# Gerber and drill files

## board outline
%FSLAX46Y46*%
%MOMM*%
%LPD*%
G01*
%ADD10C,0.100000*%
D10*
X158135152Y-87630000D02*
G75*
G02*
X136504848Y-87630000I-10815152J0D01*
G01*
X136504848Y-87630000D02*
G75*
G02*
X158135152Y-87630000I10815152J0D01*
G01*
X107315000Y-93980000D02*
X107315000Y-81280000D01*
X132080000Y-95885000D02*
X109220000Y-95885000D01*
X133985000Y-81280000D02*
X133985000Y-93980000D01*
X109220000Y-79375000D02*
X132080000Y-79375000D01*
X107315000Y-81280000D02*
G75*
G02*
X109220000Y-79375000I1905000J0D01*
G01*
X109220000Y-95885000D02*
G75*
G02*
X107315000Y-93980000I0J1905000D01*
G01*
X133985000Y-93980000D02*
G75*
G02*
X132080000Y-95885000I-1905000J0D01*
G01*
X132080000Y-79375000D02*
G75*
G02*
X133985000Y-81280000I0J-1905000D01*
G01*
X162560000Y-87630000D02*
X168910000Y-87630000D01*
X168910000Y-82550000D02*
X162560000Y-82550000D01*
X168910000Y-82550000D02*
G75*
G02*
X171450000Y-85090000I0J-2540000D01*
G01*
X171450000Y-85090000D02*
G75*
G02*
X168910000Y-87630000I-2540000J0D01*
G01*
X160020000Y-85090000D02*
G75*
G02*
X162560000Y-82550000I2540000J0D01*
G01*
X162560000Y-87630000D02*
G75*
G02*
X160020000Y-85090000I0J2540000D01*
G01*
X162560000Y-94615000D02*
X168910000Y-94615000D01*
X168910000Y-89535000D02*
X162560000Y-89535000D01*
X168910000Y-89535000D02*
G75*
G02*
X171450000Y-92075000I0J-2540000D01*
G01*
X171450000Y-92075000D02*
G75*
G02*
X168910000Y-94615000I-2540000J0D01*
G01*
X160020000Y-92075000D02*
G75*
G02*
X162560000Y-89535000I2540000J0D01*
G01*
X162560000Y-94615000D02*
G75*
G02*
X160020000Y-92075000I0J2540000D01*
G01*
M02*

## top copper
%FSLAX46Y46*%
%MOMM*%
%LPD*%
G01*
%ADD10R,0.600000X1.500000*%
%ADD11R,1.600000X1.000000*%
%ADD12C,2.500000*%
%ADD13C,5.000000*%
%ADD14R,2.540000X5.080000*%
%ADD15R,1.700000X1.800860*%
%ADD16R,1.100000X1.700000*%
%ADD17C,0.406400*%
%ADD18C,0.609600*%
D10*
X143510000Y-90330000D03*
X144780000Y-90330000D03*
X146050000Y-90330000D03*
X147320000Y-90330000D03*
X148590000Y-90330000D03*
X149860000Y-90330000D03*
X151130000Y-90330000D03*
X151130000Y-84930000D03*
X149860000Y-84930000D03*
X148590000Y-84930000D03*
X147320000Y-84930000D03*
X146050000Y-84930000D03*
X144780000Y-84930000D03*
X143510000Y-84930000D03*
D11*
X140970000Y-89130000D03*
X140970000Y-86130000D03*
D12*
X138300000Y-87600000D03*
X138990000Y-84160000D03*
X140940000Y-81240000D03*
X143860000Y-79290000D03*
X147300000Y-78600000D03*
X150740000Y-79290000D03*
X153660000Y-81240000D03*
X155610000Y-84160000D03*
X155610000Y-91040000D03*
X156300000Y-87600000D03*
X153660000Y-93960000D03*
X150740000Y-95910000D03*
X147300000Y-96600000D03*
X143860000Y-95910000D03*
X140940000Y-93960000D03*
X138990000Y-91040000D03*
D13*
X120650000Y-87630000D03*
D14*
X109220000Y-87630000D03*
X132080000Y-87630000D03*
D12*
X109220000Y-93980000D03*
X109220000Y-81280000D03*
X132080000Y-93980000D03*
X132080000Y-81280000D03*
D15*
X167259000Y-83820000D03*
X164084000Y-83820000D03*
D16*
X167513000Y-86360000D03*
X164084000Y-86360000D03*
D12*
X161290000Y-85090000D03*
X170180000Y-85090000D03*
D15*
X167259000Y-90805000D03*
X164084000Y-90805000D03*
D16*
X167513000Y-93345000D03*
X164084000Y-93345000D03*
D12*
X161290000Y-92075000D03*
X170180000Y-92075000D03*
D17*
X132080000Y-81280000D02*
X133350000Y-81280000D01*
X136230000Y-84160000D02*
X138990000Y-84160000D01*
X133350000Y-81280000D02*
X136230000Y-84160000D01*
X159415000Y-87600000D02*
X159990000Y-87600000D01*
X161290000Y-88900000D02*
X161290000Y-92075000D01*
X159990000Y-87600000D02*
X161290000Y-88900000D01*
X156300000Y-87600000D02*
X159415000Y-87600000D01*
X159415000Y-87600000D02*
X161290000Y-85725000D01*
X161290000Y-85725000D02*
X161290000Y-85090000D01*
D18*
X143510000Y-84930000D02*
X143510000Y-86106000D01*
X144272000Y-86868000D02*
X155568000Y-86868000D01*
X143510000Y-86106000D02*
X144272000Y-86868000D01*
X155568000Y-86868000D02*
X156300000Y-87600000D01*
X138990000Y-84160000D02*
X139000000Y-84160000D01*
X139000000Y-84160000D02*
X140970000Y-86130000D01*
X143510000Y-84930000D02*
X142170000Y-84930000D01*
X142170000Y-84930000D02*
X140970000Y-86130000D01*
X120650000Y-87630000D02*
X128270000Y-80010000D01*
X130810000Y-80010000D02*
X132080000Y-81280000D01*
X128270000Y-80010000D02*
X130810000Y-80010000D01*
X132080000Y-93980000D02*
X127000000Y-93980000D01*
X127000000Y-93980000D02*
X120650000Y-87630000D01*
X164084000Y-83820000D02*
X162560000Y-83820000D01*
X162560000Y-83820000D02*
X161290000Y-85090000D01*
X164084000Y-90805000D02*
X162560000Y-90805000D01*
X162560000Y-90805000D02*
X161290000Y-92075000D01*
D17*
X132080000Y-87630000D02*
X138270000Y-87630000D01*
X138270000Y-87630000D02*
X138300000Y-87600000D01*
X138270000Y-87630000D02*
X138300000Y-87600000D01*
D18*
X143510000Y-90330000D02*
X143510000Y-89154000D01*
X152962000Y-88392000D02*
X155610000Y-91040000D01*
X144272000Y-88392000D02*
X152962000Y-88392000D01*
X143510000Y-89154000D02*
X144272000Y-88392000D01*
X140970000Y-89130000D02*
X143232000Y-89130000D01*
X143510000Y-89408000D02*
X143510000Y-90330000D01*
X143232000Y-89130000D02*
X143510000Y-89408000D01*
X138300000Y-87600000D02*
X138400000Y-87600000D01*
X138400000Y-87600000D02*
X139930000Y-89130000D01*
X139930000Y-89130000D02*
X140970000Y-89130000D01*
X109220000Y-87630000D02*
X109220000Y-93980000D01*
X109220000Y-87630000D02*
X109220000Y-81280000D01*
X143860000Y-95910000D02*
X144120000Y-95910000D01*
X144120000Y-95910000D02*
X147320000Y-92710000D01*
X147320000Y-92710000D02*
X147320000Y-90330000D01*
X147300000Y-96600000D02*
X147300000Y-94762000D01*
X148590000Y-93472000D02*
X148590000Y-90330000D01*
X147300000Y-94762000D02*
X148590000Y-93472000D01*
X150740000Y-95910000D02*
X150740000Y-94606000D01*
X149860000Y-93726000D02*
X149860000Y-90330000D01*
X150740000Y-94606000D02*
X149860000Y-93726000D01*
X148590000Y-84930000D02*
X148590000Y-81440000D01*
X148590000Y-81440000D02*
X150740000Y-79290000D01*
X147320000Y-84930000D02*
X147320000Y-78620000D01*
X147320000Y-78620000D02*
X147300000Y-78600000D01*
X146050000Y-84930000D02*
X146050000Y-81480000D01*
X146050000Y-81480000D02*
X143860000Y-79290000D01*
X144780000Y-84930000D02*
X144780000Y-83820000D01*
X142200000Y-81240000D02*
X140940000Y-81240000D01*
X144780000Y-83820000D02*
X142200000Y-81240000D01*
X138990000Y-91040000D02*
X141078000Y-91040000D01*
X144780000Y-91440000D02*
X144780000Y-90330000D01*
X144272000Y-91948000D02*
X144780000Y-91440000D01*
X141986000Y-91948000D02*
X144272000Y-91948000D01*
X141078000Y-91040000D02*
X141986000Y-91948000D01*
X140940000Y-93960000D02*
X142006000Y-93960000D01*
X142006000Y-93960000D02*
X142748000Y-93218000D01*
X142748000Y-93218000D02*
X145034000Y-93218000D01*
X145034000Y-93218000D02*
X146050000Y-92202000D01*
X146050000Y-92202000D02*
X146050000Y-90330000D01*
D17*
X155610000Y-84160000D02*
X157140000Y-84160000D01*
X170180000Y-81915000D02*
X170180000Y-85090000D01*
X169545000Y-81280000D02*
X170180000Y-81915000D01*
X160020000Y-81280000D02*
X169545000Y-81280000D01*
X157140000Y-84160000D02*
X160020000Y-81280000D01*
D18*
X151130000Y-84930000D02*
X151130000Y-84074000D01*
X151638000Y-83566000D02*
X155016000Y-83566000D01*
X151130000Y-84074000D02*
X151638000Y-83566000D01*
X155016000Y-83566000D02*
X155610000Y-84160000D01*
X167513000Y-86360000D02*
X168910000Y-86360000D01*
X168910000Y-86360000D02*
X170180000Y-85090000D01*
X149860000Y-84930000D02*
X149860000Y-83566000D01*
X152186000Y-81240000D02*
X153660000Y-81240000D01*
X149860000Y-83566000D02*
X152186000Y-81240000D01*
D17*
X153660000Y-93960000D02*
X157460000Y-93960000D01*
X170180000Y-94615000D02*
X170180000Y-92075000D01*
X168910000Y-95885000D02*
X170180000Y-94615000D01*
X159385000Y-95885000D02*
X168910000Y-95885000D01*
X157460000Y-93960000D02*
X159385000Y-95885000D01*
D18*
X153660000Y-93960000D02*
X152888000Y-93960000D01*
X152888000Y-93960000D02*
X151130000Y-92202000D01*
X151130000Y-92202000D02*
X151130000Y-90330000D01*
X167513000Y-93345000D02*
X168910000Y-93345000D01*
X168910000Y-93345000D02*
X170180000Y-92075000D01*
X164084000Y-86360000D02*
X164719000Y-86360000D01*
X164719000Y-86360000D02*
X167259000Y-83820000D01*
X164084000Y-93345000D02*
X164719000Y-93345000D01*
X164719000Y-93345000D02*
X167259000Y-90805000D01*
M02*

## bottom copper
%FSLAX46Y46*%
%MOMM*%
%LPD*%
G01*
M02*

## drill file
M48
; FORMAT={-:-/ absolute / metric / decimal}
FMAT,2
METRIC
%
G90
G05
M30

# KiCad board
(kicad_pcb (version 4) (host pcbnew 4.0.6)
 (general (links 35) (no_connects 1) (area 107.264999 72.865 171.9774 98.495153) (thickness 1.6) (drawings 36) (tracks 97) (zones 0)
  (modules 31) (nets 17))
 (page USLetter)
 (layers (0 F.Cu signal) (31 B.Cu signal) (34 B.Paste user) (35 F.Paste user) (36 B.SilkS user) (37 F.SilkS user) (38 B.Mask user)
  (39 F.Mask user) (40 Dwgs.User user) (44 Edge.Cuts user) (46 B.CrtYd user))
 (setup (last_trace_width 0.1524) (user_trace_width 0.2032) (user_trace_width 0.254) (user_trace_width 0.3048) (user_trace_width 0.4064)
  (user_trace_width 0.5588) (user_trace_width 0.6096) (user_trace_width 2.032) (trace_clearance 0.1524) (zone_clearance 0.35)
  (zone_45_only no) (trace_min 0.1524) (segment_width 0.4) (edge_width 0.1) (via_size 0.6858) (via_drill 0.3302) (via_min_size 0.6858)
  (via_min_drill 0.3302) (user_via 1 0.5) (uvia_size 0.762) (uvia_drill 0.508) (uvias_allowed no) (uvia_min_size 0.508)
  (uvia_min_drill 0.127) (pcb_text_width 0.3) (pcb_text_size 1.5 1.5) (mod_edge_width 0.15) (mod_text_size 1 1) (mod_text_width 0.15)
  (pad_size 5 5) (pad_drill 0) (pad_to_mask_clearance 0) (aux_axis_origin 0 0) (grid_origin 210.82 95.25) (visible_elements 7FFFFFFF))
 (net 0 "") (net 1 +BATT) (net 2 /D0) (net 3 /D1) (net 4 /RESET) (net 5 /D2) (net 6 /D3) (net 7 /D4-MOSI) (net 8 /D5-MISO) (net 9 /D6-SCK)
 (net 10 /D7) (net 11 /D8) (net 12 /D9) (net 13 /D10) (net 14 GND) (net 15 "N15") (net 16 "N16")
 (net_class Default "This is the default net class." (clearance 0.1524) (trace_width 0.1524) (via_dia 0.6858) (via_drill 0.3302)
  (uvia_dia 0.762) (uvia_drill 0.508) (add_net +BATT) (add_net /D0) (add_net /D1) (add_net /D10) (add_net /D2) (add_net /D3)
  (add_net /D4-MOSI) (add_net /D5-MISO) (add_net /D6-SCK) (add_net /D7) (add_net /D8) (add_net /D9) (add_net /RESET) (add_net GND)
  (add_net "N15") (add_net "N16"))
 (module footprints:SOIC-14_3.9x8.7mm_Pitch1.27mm (layer F.Cu) (at 147.32 87.63 90)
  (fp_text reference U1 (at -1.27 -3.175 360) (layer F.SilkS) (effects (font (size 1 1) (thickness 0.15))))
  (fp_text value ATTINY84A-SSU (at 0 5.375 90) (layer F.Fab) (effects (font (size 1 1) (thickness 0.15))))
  (pad 1 smd rect (at -2.7 -3.81 90) (size 1.5 0.6) (layers F.Cu F.Paste F.Mask) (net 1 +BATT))
  (pad 2 smd rect (at -2.7 -2.54 90) (size 1.5 0.6) (layers F.Cu F.Paste F.Mask) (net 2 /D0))
  (pad 3 smd rect (at -2.7 -1.27 90) (size 1.5 0.6) (layers F.Cu F.Paste F.Mask) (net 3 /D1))
  (pad 4 smd rect (at -2.7 0 90) (size 1.5 0.6) (layers F.Cu F.Paste F.Mask) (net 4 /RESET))
  (pad 5 smd rect (at -2.7 1.27 90) (size 1.5 0.6) (layers F.Cu F.Paste F.Mask) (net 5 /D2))
  (pad 6 smd rect (at -2.7 2.54 90) (size 1.5 0.6) (layers F.Cu F.Paste F.Mask) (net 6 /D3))
  (pad 7 smd rect (at -2.7 3.81 90) (size 1.5 0.6) (layers F.Cu F.Paste F.Mask) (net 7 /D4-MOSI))
  (pad 8 smd rect (at 2.7 3.81 90) (size 1.5 0.6) (layers F.Cu F.Paste F.Mask) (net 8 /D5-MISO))
  (pad 9 smd rect (at 2.7 2.54 90) (size 1.5 0.6) (layers F.Cu F.Paste F.Mask) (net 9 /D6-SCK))
  (pad 10 smd rect (at 2.7 1.27 90) (size 1.5 0.6) (layers F.Cu F.Paste F.Mask) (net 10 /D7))
  (pad 11 smd rect (at 2.7 0 90) (size 1.5 0.6) (layers F.Cu F.Paste F.Mask) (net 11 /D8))
  (pad 12 smd rect (at 2.7 -1.27 90) (size 1.5 0.6) (layers F.Cu F.Paste F.Mask) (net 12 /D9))
  (pad 13 smd rect (at 2.7 -2.54 90) (size 1.5 0.6) (layers F.Cu F.Paste F.Mask) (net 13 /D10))
  (pad 14 smd rect (at 2.7 -3.81 90) (size 1.5 0.6) (layers F.Cu F.Paste F.Mask) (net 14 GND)))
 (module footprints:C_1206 (layer F.Cu) (at 140.97 87.63 90)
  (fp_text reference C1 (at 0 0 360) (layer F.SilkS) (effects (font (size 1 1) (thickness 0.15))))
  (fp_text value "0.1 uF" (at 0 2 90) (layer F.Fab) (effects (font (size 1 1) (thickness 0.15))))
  (pad 1 smd rect (at -1.5 0 90) (size 1 1.6) (layers F.Cu F.Paste F.Mask) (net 1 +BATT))
  (pad 2 smd rect (at 1.5 0 90) (size 1 1.6) (layers F.Cu F.Paste F.Mask) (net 14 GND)))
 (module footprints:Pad (layer F.Cu) (at 138.3 87.6)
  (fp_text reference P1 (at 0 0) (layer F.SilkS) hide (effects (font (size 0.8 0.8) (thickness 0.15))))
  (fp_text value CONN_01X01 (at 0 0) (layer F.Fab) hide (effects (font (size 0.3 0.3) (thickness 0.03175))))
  (pad 1 smd circle (at 0 0) (size 2.5 2.5) (layers F.Cu F.Paste F.Mask) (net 1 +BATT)))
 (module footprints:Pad (layer F.Cu) (at 138.99 84.16)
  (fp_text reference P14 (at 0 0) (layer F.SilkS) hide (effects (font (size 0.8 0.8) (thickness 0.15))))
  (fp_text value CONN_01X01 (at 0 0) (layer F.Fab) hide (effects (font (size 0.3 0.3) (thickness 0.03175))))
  (pad 1 smd circle (at 0 0) (size 2.5 2.5) (layers F.Cu F.Paste F.Mask) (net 14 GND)))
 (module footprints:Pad (layer F.Cu) (at 140.94 81.24)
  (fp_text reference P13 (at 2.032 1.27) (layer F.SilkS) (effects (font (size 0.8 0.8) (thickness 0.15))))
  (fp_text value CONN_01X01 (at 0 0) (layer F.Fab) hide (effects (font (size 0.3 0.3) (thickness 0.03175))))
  (pad 1 smd circle (at 0 0) (size 2.5 2.5) (layers F.Cu F.Paste F.Mask) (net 13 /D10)))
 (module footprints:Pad (layer F.Cu) (at 143.86 79.29)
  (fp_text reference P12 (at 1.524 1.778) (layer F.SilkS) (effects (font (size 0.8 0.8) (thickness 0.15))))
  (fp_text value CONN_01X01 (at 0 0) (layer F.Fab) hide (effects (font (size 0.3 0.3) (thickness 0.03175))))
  (pad 1 smd circle (at 0 0) (size 2.5 2.5) (layers F.Cu F.Paste F.Mask) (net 12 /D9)))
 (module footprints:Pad (layer F.Cu) (at 147.3 78.6)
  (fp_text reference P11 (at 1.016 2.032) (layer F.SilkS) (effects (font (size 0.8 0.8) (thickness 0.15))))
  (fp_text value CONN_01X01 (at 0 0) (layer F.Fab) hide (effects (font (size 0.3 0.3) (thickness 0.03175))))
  (pad 1 smd circle (at 0 0) (size 2.5 2.5) (layers F.Cu F.Paste F.Mask) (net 11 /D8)))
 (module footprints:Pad (layer F.Cu) (at 150.74 79.29)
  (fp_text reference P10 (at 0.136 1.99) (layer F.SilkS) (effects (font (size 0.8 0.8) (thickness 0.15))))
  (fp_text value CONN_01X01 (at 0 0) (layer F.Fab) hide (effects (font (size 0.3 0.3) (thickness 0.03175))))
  (pad 1 smd circle (at 0 0) (size 2.5 2.5) (layers F.Cu F.Paste F.Mask) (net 10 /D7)))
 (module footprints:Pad (layer F.Cu) (at 153.66 81.24)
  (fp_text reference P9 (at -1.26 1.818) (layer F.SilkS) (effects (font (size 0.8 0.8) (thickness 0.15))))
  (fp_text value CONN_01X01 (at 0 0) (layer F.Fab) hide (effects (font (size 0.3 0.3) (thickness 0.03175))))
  (pad 1 smd circle (at 0 0) (size 2.5 2.5) (layers F.Cu F.Paste F.Mask) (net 9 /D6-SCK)))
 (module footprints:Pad (layer F.Cu) (at 155.61 84.16)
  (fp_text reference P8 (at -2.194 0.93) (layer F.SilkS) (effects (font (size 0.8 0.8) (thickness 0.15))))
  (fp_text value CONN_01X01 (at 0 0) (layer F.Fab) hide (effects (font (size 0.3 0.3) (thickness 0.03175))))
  (pad 1 smd circle (at 0 0) (size 2.5 2.5) (layers F.Cu F.Paste F.Mask) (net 8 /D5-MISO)))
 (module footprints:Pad (layer F.Cu) (at 155.61 91.04)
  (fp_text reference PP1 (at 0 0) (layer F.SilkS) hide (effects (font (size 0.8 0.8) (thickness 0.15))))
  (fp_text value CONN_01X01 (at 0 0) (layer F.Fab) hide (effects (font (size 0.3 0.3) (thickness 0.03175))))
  (pad 1 smd circle (at 0 0) (size 2.5 2.5) (layers F.Cu F.Paste F.Mask) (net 1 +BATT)))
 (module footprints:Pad (layer F.Cu) (at 156.3 87.6)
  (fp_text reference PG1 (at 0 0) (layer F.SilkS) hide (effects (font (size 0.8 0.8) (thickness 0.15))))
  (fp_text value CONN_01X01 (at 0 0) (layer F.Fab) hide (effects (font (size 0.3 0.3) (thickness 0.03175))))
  (pad 1 smd circle (at 0 0) (size 2.5 2.5) (layers F.Cu F.Paste F.Mask) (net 14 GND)))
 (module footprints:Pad (layer F.Cu) (at 153.66 93.96)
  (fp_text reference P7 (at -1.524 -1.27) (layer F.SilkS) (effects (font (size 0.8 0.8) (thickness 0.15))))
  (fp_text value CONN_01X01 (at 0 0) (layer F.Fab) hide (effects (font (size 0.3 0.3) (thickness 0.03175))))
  (pad 1 smd circle (at 0 0) (size 2.5 2.5) (layers F.Cu F.Paste F.Mask) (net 7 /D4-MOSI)))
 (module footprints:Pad (layer F.Cu) (at 150.74 95.91)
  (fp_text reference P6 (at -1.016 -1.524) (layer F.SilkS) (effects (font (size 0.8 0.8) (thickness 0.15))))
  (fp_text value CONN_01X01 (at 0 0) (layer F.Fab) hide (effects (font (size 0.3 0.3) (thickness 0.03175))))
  (pad 1 smd circle (at 0 0) (size 2.5 2.5) (layers F.Cu F.Paste F.Mask) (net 6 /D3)))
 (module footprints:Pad (layer F.Cu) (at 147.3 96.6)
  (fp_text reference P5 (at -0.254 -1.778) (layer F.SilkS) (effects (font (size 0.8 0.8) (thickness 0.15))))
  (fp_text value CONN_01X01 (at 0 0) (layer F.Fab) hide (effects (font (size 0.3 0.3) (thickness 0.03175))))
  (pad 1 smd circle (at 0 0) (size 2.5 2.5) (layers F.Cu F.Paste F.Mask) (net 5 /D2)))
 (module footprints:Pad (layer F.Cu) (at 143.86 95.91)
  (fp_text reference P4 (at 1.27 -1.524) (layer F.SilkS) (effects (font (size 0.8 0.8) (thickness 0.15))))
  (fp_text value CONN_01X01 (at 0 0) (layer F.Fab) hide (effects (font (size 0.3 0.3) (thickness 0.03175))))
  (pad 1 smd circle (at 0 0) (size 2.5 2.5) (layers F.Cu F.Paste F.Mask) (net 4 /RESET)))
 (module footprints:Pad (layer F.Cu) (at 140.94 93.96)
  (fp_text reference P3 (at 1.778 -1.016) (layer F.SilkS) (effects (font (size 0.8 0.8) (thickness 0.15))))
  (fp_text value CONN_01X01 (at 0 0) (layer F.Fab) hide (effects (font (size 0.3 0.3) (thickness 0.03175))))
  (pad 1 smd circle (at 0 0) (size 2.5 2.5) (layers F.Cu F.Paste F.Mask) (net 3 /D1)))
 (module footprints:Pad (layer F.Cu) (at 138.99 91.04)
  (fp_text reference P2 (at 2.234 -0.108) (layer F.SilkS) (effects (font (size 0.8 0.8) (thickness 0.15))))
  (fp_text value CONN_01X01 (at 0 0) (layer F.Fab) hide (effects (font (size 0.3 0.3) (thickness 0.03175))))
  (pad 1 smd circle (at 0 0) (size 2.5 2.5) (layers F.Cu F.Paste F.Mask) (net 2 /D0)))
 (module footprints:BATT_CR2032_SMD (layer F.Cu) (at 120.65 87.63)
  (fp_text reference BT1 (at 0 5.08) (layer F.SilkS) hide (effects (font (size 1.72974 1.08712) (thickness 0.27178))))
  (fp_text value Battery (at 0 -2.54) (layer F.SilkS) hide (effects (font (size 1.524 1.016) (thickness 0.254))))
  (pad 2 smd circle (at 0 0) (size 5 5) (layers F.Cu F.Paste F.Mask) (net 14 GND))
  (pad 1 smd rect (at -11.43 0) (size 2.54 5.08) (layers F.Cu F.Paste F.Mask) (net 1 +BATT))
  (pad 1 smd rect (at 11.43 0) (size 2.54 5.08) (layers F.Cu F.Paste F.Mask) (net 1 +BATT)))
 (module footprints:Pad (layer F.Cu) (at 109.22 93.98)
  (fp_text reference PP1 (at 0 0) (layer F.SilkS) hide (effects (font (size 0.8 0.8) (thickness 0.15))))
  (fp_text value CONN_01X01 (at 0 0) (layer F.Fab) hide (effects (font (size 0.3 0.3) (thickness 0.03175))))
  (pad 1 smd circle (at 0 0) (size 2.5 2.5) (layers F.Cu F.Paste F.Mask) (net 1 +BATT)))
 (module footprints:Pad (layer F.Cu) (at 109.22 81.28)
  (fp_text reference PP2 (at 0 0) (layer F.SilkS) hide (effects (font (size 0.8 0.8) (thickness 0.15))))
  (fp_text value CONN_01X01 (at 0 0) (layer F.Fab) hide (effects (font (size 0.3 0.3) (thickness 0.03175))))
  (pad 1 smd circle (at 0 0) (size 2.5 2.5) (layers F.Cu F.Paste F.Mask) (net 1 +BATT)))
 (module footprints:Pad (layer F.Cu) (at 132.08 93.98)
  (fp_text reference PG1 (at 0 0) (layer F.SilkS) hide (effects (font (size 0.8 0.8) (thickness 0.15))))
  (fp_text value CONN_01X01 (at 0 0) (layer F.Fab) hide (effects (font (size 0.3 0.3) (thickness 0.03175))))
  (pad 1 smd circle (at 0 0) (size 2.5 2.5) (layers F.Cu F.Paste F.Mask) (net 14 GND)))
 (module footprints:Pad (layer F.Cu) (at 132.08 81.28)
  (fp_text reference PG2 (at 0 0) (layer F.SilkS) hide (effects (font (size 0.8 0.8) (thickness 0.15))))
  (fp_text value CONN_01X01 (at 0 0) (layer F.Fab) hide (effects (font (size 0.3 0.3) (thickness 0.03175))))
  (pad 1 smd circle (at 0 0) (size 2.5 2.5) (layers F.Cu F.Paste F.Mask) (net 14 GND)))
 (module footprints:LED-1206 (layer F.Cu) (at 165.735 83.82)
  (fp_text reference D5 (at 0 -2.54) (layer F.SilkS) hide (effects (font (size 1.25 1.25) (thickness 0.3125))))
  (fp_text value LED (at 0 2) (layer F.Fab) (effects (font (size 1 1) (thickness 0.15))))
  (pad 2 smd rect (at 1.524 0 180) (size 1.7 1.80086) (layers F.Cu F.Paste F.Mask) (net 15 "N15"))
  (pad 1 smd rect (at -1.651 0 180) (size 1.7 1.80086) (layers F.Cu F.Paste F.Mask) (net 14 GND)))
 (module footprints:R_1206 (layer F.Cu) (at 165.735 86.36 180)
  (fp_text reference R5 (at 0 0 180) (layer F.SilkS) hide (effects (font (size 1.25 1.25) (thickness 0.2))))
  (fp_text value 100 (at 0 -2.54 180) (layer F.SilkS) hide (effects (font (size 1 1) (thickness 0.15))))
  (pad 1 smd rect (at -1.778 0 180) (size 1.1 1.7) (layers F.Cu F.Paste F.Mask) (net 8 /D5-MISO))
  (pad 2 smd rect (at 1.651 0 180) (size 1.1 1.7) (layers F.Cu F.Paste F.Mask) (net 15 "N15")))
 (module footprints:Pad (layer F.Cu) (at 161.29 85.09 90)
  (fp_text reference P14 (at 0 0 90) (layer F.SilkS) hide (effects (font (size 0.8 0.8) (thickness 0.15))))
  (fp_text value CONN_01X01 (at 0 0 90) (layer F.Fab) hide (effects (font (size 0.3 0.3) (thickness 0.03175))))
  (pad 1 smd circle (at 0 0 90) (size 2.5 2.5) (layers F.Cu F.Paste F.Mask) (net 14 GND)))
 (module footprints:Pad (layer F.Cu) (at 170.18 85.09 90)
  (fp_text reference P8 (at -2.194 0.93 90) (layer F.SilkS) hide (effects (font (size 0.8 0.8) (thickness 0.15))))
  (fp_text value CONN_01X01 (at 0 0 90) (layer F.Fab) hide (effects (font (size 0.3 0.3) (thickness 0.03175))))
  (pad 1 smd circle (at 0 0 90) (size 2.5 2.5) (layers F.Cu F.Paste F.Mask) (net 8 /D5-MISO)))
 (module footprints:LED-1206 (layer F.Cu) (at 165.735 90.805)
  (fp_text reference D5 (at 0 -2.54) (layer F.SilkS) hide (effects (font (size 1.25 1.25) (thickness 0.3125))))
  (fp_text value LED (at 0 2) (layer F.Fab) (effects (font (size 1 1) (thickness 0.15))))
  (pad 2 smd rect (at 1.524 0 180) (size 1.7 1.80086) (layers F.Cu F.Paste F.Mask) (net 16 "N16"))
  (pad 1 smd rect (at -1.651 0 180) (size 1.7 1.80086) (layers F.Cu F.Paste F.Mask) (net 14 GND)))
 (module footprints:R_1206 (layer F.Cu) (at 165.735 93.345 180)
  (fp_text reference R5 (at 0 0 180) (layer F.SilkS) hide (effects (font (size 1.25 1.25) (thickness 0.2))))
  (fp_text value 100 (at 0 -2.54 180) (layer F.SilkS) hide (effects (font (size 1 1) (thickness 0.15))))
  (pad 1 smd rect (at -1.778 0 180) (size 1.1 1.7) (layers F.Cu F.Paste F.Mask) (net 7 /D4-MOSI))
  (pad 2 smd rect (at 1.651 0 180) (size 1.1 1.7) (layers F.Cu F.Paste F.Mask) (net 16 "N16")))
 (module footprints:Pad (layer F.Cu) (at 161.29 92.075 90)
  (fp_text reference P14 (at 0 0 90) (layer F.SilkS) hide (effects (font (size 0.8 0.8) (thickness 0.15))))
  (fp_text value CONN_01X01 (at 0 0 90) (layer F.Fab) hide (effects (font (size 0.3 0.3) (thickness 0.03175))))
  (pad 1 smd circle (at 0 0 90) (size 2.5 2.5) (layers F.Cu F.Paste F.Mask) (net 14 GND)))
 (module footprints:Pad (layer F.Cu) (at 170.18 92.075 90)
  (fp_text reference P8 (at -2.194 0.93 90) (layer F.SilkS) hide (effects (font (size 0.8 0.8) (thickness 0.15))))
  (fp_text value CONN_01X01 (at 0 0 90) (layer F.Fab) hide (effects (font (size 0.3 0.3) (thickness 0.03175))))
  (pad 1 smd circle (at 0 0 90) (size 2.5 2.5) (layers F.Cu F.Paste F.Mask) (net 7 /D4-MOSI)))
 (gr_circle (center 147.32 87.63) (end 149.098 98.298) (layer Edge.Cuts) (width 0.1))
 (gr_line (start 107.315 93.98) (end 107.315 81.28) (angle 90) (layer Edge.Cuts) (width 0.1))
 (gr_line (start 132.08 95.885) (end 109.22 95.885) (angle 90) (layer Edge.Cuts) (width 0.1))
 (gr_line (start 133.985 81.28) (end 133.985 93.98) (angle 90) (layer Edge.Cuts) (width 0.1))
 (gr_line (start 109.22 79.375) (end 132.08 79.375) (angle 90) (layer Edge.Cuts) (width 0.1))
 (gr_arc (start 109.22 81.28) (end 107.315 81.28) (angle 90) (layer Edge.Cuts) (width 0.1))
 (gr_arc (start 109.22 93.98) (end 109.22 95.885) (angle 90) (layer Edge.Cuts) (width 0.1))
 (gr_arc (start 132.08 93.98) (end 133.985 93.98) (angle 90) (layer Edge.Cuts) (width 0.1))
 (gr_arc (start 132.08 81.28) (end 132.08 79.375) (angle 90) (layer Edge.Cuts) (width 0.1))
 (gr_line (start 162.56 87.63) (end 168.91 87.63) (angle 90) (layer Edge.Cuts) (width 0.1))
 (gr_line (start 168.91 82.55) (end 162.56 82.55) (angle 90) (layer Edge.Cuts) (width 0.1))
 (gr_arc (start 168.91 85.09) (end 168.91 82.55) (angle 90) (layer Edge.Cuts) (width 0.1))
 (gr_arc (start 168.91 85.09) (end 171.45 85.09) (angle 90) (layer Edge.Cuts) (width 0.1))
 (gr_arc (start 162.56 85.09) (end 160.02 85.09) (angle 90) (layer Edge.Cuts) (width 0.1))
 (gr_arc (start 162.56 85.09) (end 162.56 87.63) (angle 90) (layer Edge.Cuts) (width 0.1))
 (gr_line (start 162.56 94.615) (end 168.91 94.615) (angle 90) (layer Edge.Cuts) (width 0.1))
 (gr_line (start 168.91 89.535) (end 162.56 89.535) (angle 90) (layer Edge.Cuts) (width 0.1))
 (gr_arc (start 168.91 92.075) (end 168.91 89.535) (angle 90) (layer Edge.Cuts) (width 0.1))
 (gr_arc (start 168.91 92.075) (end 171.45 92.075) (angle 90) (layer Edge.Cuts) (width 0.1))
 (gr_arc (start 162.56 92.075) (end 160.02 92.075) (angle 90) (layer Edge.Cuts) (width 0.1))
 (gr_arc (start 162.56 92.075) (end 162.56 94.615) (angle 90) (layer Edge.Cuts) (width 0.1))
 (segment (start 132.08 81.28) (end 133.35 81.28) (width 0.4064) (layer F.Cu) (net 14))
 (segment (start 136.23 84.16) (end 138.99 84.16) (width 0.4064) (layer F.Cu) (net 14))
 (segment (start 133.35 81.28) (end 136.23 84.16) (width 0.4064) (layer F.Cu) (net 14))
 (segment (start 159.415 87.6) (end 159.99 87.6) (width 0.4064) (layer F.Cu) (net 14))
 (segment (start 161.29 88.9) (end 161.29 92.075) (width 0.4064) (layer F.Cu) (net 14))
 (segment (start 159.99 87.6) (end 161.29 88.9) (width 0.4064) (layer F.Cu) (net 14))
 (segment (start 156.3 87.6) (end 159.415 87.6) (width 0.4064) (layer F.Cu) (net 14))
 (segment (start 159.415 87.6) (end 161.29 85.725) (width 0.4064) (layer F.Cu) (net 14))
 (segment (start 161.29 85.725) (end 161.29 85.09) (width 0.4064) (layer F.Cu) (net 14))
 (segment (start 143.51 84.93) (end 143.51 86.106) (width 0.6096) (layer F.Cu) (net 14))
 (segment (start 144.272 86.868) (end 155.568 86.868) (width 0.6096) (layer F.Cu) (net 14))
 (segment (start 143.51 86.106) (end 144.272 86.868) (width 0.6096) (layer F.Cu) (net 14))
 (segment (start 155.568 86.868) (end 156.3 87.6) (width 0.6096) (layer F.Cu) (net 14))
 (segment (start 138.99 84.16) (end 139 84.16) (width 0.6096) (layer F.Cu) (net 14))
 (segment (start 139 84.16) (end 140.97 86.13) (width 0.6096) (layer F.Cu) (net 14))
 (segment (start 143.51 84.93) (end 142.17 84.93) (width 0.6096) (layer F.Cu) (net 14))
 (segment (start 142.17 84.93) (end 140.97 86.13) (width 0.6096) (layer F.Cu) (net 14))
 (segment (start 120.65 87.63) (end 128.27 80.01) (width 0.6096) (layer F.Cu) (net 14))
 (segment (start 130.81 80.01) (end 132.08 81.28) (width 0.6096) (layer F.Cu) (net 14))
 (segment (start 128.27 80.01) (end 130.81 80.01) (width 0.6096) (layer F.Cu) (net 14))
 (segment (start 132.08 93.98) (end 127 93.98) (width 0.6096) (layer F.Cu) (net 14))
 (segment (start 127 93.98) (end 120.65 87.63) (width 0.6096) (layer F.Cu) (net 14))
 (segment (start 164.084 83.82) (end 162.56 83.82) (width 0.6096) (layer F.Cu) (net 14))
 (segment (start 162.56 83.82) (end 161.29 85.09) (width 0.6096) (layer F.Cu) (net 14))
 (segment (start 164.084 90.805) (end 162.56 90.805) (width 0.6096) (layer F.Cu) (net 14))
 (segment (start 162.56 90.805) (end 161.29 92.075) (width 0.6096) (layer F.Cu) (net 14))
 (segment (start 132.08 87.63) (end 138.27 87.63) (width 0.4064) (layer F.Cu) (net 1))
 (segment (start 138.27 87.63) (end 138.3 87.6) (width 0.4064) (layer F.Cu) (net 1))
 (segment (start 138.27 87.63) (end 138.3 87.6) (width 0.4064) (layer F.Cu) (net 1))
 (segment (start 143.51 90.33) (end 143.51 89.154) (width 0.6096) (layer F.Cu) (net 1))
 (segment (start 152.962 88.392) (end 155.61 91.04) (width 0.6096) (layer F.Cu) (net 1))
 (segment (start 144.272 88.392) (end 152.962 88.392) (width 0.6096) (layer F.Cu) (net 1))
 (segment (start 143.51 89.154) (end 144.272 88.392) (width 0.6096) (layer F.Cu) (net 1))
 (segment (start 140.97 89.13) (end 143.232 89.13) (width 0.6096) (layer F.Cu) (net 1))
 (segment (start 143.51 89.408) (end 143.51 90.33) (width 0.6096) (layer F.Cu) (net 1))
 (segment (start 143.232 89.13) (end 143.51 89.408) (width 0.6096) (layer F.Cu) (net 1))
 (segment (start 138.3 87.6) (end 138.4 87.6) (width 0.6096) (layer F.Cu) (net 1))
 (segment (start 138.4 87.6) (end 139.93 89.13) (width 0.6096) (layer F.Cu) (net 1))
 (segment (start 139.93 89.13) (end 140.97 89.13) (width 0.6096) (layer F.Cu) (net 1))
 (segment (start 109.22 87.63) (end 109.22 93.98) (width 0.6096) (layer F.Cu) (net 1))
 (segment (start 109.22 87.63) (end 109.22 81.28) (width 0.6096) (layer F.Cu) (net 1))
 (segment (start 143.86 95.91) (end 144.12 95.91) (width 0.6096) (layer F.Cu) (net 4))
 (segment (start 144.12 95.91) (end 147.32 92.71) (width 0.6096) (layer F.Cu) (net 4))
 (segment (start 147.32 92.71) (end 147.32 90.33) (width 0.6096) (layer F.Cu) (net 4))
 (segment (start 147.3 96.6) (end 147.3 94.762) (width 0.6096) (layer F.Cu) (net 5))
 (segment (start 148.59 93.472) (end 148.59 90.33) (width 0.6096) (layer F.Cu) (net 5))
 (segment (start 147.3 94.762) (end 148.59 93.472) (width 0.6096) (layer F.Cu) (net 5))
 (segment (start 150.74 95.91) (end 150.74 94.606) (width 0.6096) (layer F.Cu) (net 6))
 (segment (start 149.86 93.726) (end 149.86 90.33) (width 0.6096) (layer F.Cu) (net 6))
 (segment (start 150.74 94.606) (end 149.86 93.726) (width 0.6096) (layer F.Cu) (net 6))
 (segment (start 148.59 84.93) (end 148.59 81.44) (width 0.6096) (layer F.Cu) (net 10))
 (segment (start 148.59 81.44) (end 150.74 79.29) (width 0.6096) (layer F.Cu) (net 10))
 (segment (start 147.32 84.93) (end 147.32 78.62) (width 0.6096) (layer F.Cu) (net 11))
 (segment (start 147.32 78.62) (end 147.3 78.6) (width 0.6096) (layer F.Cu) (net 11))
 (segment (start 146.05 84.93) (end 146.05 81.48) (width 0.6096) (layer F.Cu) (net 12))
 (segment (start 146.05 81.48) (end 143.86 79.29) (width 0.6096) (layer F.Cu) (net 12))
 (segment (start 144.78 84.93) (end 144.78 83.82) (width 0.6096) (layer F.Cu) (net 13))
 (segment (start 142.2 81.24) (end 140.94 81.24) (width 0.6096) (layer F.Cu) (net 13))
 (segment (start 144.78 83.82) (end 142.2 81.24) (width 0.6096) (layer F.Cu) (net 13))
 (segment (start 138.99 91.04) (end 141.078 91.04) (width 0.6096) (layer F.Cu) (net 2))
 (segment (start 144.78 91.44) (end 144.78 90.33) (width 0.6096) (layer F.Cu) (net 2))
 (segment (start 144.272 91.948) (end 144.78 91.44) (width 0.6096) (layer F.Cu) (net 2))
 (segment (start 141.986 91.948) (end 144.272 91.948) (width 0.6096) (layer F.Cu) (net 2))
 (segment (start 141.078 91.04) (end 141.986 91.948) (width 0.6096) (layer F.Cu) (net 2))
 (segment (start 140.94 93.96) (end 142.006 93.96) (width 0.6096) (layer F.Cu) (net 3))
 (segment (start 142.006 93.96) (end 142.748 93.218) (width 0.6096) (layer F.Cu) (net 3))
 (segment (start 142.748 93.218) (end 145.034 93.218) (width 0.6096) (layer F.Cu) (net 3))
 (segment (start 145.034 93.218) (end 146.05 92.202) (width 0.6096) (layer F.Cu) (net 3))
 (segment (start 146.05 92.202) (end 146.05 90.33) (width 0.6096) (layer F.Cu) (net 3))
 (segment (start 155.61 84.16) (end 157.14 84.16) (width 0.4064) (layer F.Cu) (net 8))
 (segment (start 170.18 81.915) (end 170.18 85.09) (width 0.4064) (layer F.Cu) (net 8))
 (segment (start 169.545 81.28) (end 170.18 81.915) (width 0.4064) (layer F.Cu) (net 8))
 (segment (start 160.02 81.28) (end 169.545 81.28) (width 0.4064) (layer F.Cu) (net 8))
 (segment (start 157.14 84.16) (end 160.02 81.28) (width 0.4064) (layer F.Cu) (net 8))
 (segment (start 151.13 84.93) (end 151.13 84.074) (width 0.6096) (layer F.Cu) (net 8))
 (segment (start 151.638 83.566) (end 155.016 83.566) (width 0.6096) (layer F.Cu) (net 8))
 (segment (start 151.13 84.074) (end 151.638 83.566) (width 0.6096) (layer F.Cu) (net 8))
 (segment (start 155.016 83.566) (end 155.61 84.16) (width 0.6096) (layer F.Cu) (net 8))
 (segment (start 167.513 86.36) (end 168.91 86.36) (width 0.6096) (layer F.Cu) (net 8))
 (segment (start 168.91 86.36) (end 170.18 85.09) (width 0.6096) (layer F.Cu) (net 8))
 (segment (start 149.86 84.93) (end 149.86 83.566) (width 0.6096) (layer F.Cu) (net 9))
 (segment (start 152.186 81.24) (end 153.66 81.24) (width 0.6096) (layer F.Cu) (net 9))
 (segment (start 149.86 83.566) (end 152.186 81.24) (width 0.6096) (layer F.Cu) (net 9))
 (segment (start 153.66 93.96) (end 157.46 93.96) (width 0.4064) (layer F.Cu) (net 7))
 (segment (start 170.18 94.615) (end 170.18 92.075) (width 0.4064) (layer F.Cu) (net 7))
 (segment (start 168.91 95.885) (end 170.18 94.615) (width 0.4064) (layer F.Cu) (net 7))
 (segment (start 159.385 95.885) (end 168.91 95.885) (width 0.4064) (layer F.Cu) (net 7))
 (segment (start 157.46 93.96) (end 159.385 95.885) (width 0.4064) (layer F.Cu) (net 7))
 (segment (start 153.66 93.96) (end 152.888 93.96) (width 0.6096) (layer F.Cu) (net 7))
 (segment (start 152.888 93.96) (end 151.13 92.202) (width 0.6096) (layer F.Cu) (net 7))
 (segment (start 151.13 92.202) (end 151.13 90.33) (width 0.6096) (layer F.Cu) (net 7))
 (segment (start 167.513 93.345) (end 168.91 93.345) (width 0.6096) (layer F.Cu) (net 7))
 (segment (start 168.91 93.345) (end 170.18 92.075) (width 0.6096) (layer F.Cu) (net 7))
 (segment (start 164.084 86.36) (end 164.719 86.36) (width 0.6096) (layer F.Cu) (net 15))
 (segment (start 164.719 86.36) (end 167.259 83.82) (width 0.6096) (layer F.Cu) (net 15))
 (segment (start 164.084 93.345) (end 164.719 93.345) (width 0.6096) (layer F.Cu) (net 16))
 (segment (start 164.719 93.345) (end 167.259 90.805) (width 0.6096) (layer F.Cu) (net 16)))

